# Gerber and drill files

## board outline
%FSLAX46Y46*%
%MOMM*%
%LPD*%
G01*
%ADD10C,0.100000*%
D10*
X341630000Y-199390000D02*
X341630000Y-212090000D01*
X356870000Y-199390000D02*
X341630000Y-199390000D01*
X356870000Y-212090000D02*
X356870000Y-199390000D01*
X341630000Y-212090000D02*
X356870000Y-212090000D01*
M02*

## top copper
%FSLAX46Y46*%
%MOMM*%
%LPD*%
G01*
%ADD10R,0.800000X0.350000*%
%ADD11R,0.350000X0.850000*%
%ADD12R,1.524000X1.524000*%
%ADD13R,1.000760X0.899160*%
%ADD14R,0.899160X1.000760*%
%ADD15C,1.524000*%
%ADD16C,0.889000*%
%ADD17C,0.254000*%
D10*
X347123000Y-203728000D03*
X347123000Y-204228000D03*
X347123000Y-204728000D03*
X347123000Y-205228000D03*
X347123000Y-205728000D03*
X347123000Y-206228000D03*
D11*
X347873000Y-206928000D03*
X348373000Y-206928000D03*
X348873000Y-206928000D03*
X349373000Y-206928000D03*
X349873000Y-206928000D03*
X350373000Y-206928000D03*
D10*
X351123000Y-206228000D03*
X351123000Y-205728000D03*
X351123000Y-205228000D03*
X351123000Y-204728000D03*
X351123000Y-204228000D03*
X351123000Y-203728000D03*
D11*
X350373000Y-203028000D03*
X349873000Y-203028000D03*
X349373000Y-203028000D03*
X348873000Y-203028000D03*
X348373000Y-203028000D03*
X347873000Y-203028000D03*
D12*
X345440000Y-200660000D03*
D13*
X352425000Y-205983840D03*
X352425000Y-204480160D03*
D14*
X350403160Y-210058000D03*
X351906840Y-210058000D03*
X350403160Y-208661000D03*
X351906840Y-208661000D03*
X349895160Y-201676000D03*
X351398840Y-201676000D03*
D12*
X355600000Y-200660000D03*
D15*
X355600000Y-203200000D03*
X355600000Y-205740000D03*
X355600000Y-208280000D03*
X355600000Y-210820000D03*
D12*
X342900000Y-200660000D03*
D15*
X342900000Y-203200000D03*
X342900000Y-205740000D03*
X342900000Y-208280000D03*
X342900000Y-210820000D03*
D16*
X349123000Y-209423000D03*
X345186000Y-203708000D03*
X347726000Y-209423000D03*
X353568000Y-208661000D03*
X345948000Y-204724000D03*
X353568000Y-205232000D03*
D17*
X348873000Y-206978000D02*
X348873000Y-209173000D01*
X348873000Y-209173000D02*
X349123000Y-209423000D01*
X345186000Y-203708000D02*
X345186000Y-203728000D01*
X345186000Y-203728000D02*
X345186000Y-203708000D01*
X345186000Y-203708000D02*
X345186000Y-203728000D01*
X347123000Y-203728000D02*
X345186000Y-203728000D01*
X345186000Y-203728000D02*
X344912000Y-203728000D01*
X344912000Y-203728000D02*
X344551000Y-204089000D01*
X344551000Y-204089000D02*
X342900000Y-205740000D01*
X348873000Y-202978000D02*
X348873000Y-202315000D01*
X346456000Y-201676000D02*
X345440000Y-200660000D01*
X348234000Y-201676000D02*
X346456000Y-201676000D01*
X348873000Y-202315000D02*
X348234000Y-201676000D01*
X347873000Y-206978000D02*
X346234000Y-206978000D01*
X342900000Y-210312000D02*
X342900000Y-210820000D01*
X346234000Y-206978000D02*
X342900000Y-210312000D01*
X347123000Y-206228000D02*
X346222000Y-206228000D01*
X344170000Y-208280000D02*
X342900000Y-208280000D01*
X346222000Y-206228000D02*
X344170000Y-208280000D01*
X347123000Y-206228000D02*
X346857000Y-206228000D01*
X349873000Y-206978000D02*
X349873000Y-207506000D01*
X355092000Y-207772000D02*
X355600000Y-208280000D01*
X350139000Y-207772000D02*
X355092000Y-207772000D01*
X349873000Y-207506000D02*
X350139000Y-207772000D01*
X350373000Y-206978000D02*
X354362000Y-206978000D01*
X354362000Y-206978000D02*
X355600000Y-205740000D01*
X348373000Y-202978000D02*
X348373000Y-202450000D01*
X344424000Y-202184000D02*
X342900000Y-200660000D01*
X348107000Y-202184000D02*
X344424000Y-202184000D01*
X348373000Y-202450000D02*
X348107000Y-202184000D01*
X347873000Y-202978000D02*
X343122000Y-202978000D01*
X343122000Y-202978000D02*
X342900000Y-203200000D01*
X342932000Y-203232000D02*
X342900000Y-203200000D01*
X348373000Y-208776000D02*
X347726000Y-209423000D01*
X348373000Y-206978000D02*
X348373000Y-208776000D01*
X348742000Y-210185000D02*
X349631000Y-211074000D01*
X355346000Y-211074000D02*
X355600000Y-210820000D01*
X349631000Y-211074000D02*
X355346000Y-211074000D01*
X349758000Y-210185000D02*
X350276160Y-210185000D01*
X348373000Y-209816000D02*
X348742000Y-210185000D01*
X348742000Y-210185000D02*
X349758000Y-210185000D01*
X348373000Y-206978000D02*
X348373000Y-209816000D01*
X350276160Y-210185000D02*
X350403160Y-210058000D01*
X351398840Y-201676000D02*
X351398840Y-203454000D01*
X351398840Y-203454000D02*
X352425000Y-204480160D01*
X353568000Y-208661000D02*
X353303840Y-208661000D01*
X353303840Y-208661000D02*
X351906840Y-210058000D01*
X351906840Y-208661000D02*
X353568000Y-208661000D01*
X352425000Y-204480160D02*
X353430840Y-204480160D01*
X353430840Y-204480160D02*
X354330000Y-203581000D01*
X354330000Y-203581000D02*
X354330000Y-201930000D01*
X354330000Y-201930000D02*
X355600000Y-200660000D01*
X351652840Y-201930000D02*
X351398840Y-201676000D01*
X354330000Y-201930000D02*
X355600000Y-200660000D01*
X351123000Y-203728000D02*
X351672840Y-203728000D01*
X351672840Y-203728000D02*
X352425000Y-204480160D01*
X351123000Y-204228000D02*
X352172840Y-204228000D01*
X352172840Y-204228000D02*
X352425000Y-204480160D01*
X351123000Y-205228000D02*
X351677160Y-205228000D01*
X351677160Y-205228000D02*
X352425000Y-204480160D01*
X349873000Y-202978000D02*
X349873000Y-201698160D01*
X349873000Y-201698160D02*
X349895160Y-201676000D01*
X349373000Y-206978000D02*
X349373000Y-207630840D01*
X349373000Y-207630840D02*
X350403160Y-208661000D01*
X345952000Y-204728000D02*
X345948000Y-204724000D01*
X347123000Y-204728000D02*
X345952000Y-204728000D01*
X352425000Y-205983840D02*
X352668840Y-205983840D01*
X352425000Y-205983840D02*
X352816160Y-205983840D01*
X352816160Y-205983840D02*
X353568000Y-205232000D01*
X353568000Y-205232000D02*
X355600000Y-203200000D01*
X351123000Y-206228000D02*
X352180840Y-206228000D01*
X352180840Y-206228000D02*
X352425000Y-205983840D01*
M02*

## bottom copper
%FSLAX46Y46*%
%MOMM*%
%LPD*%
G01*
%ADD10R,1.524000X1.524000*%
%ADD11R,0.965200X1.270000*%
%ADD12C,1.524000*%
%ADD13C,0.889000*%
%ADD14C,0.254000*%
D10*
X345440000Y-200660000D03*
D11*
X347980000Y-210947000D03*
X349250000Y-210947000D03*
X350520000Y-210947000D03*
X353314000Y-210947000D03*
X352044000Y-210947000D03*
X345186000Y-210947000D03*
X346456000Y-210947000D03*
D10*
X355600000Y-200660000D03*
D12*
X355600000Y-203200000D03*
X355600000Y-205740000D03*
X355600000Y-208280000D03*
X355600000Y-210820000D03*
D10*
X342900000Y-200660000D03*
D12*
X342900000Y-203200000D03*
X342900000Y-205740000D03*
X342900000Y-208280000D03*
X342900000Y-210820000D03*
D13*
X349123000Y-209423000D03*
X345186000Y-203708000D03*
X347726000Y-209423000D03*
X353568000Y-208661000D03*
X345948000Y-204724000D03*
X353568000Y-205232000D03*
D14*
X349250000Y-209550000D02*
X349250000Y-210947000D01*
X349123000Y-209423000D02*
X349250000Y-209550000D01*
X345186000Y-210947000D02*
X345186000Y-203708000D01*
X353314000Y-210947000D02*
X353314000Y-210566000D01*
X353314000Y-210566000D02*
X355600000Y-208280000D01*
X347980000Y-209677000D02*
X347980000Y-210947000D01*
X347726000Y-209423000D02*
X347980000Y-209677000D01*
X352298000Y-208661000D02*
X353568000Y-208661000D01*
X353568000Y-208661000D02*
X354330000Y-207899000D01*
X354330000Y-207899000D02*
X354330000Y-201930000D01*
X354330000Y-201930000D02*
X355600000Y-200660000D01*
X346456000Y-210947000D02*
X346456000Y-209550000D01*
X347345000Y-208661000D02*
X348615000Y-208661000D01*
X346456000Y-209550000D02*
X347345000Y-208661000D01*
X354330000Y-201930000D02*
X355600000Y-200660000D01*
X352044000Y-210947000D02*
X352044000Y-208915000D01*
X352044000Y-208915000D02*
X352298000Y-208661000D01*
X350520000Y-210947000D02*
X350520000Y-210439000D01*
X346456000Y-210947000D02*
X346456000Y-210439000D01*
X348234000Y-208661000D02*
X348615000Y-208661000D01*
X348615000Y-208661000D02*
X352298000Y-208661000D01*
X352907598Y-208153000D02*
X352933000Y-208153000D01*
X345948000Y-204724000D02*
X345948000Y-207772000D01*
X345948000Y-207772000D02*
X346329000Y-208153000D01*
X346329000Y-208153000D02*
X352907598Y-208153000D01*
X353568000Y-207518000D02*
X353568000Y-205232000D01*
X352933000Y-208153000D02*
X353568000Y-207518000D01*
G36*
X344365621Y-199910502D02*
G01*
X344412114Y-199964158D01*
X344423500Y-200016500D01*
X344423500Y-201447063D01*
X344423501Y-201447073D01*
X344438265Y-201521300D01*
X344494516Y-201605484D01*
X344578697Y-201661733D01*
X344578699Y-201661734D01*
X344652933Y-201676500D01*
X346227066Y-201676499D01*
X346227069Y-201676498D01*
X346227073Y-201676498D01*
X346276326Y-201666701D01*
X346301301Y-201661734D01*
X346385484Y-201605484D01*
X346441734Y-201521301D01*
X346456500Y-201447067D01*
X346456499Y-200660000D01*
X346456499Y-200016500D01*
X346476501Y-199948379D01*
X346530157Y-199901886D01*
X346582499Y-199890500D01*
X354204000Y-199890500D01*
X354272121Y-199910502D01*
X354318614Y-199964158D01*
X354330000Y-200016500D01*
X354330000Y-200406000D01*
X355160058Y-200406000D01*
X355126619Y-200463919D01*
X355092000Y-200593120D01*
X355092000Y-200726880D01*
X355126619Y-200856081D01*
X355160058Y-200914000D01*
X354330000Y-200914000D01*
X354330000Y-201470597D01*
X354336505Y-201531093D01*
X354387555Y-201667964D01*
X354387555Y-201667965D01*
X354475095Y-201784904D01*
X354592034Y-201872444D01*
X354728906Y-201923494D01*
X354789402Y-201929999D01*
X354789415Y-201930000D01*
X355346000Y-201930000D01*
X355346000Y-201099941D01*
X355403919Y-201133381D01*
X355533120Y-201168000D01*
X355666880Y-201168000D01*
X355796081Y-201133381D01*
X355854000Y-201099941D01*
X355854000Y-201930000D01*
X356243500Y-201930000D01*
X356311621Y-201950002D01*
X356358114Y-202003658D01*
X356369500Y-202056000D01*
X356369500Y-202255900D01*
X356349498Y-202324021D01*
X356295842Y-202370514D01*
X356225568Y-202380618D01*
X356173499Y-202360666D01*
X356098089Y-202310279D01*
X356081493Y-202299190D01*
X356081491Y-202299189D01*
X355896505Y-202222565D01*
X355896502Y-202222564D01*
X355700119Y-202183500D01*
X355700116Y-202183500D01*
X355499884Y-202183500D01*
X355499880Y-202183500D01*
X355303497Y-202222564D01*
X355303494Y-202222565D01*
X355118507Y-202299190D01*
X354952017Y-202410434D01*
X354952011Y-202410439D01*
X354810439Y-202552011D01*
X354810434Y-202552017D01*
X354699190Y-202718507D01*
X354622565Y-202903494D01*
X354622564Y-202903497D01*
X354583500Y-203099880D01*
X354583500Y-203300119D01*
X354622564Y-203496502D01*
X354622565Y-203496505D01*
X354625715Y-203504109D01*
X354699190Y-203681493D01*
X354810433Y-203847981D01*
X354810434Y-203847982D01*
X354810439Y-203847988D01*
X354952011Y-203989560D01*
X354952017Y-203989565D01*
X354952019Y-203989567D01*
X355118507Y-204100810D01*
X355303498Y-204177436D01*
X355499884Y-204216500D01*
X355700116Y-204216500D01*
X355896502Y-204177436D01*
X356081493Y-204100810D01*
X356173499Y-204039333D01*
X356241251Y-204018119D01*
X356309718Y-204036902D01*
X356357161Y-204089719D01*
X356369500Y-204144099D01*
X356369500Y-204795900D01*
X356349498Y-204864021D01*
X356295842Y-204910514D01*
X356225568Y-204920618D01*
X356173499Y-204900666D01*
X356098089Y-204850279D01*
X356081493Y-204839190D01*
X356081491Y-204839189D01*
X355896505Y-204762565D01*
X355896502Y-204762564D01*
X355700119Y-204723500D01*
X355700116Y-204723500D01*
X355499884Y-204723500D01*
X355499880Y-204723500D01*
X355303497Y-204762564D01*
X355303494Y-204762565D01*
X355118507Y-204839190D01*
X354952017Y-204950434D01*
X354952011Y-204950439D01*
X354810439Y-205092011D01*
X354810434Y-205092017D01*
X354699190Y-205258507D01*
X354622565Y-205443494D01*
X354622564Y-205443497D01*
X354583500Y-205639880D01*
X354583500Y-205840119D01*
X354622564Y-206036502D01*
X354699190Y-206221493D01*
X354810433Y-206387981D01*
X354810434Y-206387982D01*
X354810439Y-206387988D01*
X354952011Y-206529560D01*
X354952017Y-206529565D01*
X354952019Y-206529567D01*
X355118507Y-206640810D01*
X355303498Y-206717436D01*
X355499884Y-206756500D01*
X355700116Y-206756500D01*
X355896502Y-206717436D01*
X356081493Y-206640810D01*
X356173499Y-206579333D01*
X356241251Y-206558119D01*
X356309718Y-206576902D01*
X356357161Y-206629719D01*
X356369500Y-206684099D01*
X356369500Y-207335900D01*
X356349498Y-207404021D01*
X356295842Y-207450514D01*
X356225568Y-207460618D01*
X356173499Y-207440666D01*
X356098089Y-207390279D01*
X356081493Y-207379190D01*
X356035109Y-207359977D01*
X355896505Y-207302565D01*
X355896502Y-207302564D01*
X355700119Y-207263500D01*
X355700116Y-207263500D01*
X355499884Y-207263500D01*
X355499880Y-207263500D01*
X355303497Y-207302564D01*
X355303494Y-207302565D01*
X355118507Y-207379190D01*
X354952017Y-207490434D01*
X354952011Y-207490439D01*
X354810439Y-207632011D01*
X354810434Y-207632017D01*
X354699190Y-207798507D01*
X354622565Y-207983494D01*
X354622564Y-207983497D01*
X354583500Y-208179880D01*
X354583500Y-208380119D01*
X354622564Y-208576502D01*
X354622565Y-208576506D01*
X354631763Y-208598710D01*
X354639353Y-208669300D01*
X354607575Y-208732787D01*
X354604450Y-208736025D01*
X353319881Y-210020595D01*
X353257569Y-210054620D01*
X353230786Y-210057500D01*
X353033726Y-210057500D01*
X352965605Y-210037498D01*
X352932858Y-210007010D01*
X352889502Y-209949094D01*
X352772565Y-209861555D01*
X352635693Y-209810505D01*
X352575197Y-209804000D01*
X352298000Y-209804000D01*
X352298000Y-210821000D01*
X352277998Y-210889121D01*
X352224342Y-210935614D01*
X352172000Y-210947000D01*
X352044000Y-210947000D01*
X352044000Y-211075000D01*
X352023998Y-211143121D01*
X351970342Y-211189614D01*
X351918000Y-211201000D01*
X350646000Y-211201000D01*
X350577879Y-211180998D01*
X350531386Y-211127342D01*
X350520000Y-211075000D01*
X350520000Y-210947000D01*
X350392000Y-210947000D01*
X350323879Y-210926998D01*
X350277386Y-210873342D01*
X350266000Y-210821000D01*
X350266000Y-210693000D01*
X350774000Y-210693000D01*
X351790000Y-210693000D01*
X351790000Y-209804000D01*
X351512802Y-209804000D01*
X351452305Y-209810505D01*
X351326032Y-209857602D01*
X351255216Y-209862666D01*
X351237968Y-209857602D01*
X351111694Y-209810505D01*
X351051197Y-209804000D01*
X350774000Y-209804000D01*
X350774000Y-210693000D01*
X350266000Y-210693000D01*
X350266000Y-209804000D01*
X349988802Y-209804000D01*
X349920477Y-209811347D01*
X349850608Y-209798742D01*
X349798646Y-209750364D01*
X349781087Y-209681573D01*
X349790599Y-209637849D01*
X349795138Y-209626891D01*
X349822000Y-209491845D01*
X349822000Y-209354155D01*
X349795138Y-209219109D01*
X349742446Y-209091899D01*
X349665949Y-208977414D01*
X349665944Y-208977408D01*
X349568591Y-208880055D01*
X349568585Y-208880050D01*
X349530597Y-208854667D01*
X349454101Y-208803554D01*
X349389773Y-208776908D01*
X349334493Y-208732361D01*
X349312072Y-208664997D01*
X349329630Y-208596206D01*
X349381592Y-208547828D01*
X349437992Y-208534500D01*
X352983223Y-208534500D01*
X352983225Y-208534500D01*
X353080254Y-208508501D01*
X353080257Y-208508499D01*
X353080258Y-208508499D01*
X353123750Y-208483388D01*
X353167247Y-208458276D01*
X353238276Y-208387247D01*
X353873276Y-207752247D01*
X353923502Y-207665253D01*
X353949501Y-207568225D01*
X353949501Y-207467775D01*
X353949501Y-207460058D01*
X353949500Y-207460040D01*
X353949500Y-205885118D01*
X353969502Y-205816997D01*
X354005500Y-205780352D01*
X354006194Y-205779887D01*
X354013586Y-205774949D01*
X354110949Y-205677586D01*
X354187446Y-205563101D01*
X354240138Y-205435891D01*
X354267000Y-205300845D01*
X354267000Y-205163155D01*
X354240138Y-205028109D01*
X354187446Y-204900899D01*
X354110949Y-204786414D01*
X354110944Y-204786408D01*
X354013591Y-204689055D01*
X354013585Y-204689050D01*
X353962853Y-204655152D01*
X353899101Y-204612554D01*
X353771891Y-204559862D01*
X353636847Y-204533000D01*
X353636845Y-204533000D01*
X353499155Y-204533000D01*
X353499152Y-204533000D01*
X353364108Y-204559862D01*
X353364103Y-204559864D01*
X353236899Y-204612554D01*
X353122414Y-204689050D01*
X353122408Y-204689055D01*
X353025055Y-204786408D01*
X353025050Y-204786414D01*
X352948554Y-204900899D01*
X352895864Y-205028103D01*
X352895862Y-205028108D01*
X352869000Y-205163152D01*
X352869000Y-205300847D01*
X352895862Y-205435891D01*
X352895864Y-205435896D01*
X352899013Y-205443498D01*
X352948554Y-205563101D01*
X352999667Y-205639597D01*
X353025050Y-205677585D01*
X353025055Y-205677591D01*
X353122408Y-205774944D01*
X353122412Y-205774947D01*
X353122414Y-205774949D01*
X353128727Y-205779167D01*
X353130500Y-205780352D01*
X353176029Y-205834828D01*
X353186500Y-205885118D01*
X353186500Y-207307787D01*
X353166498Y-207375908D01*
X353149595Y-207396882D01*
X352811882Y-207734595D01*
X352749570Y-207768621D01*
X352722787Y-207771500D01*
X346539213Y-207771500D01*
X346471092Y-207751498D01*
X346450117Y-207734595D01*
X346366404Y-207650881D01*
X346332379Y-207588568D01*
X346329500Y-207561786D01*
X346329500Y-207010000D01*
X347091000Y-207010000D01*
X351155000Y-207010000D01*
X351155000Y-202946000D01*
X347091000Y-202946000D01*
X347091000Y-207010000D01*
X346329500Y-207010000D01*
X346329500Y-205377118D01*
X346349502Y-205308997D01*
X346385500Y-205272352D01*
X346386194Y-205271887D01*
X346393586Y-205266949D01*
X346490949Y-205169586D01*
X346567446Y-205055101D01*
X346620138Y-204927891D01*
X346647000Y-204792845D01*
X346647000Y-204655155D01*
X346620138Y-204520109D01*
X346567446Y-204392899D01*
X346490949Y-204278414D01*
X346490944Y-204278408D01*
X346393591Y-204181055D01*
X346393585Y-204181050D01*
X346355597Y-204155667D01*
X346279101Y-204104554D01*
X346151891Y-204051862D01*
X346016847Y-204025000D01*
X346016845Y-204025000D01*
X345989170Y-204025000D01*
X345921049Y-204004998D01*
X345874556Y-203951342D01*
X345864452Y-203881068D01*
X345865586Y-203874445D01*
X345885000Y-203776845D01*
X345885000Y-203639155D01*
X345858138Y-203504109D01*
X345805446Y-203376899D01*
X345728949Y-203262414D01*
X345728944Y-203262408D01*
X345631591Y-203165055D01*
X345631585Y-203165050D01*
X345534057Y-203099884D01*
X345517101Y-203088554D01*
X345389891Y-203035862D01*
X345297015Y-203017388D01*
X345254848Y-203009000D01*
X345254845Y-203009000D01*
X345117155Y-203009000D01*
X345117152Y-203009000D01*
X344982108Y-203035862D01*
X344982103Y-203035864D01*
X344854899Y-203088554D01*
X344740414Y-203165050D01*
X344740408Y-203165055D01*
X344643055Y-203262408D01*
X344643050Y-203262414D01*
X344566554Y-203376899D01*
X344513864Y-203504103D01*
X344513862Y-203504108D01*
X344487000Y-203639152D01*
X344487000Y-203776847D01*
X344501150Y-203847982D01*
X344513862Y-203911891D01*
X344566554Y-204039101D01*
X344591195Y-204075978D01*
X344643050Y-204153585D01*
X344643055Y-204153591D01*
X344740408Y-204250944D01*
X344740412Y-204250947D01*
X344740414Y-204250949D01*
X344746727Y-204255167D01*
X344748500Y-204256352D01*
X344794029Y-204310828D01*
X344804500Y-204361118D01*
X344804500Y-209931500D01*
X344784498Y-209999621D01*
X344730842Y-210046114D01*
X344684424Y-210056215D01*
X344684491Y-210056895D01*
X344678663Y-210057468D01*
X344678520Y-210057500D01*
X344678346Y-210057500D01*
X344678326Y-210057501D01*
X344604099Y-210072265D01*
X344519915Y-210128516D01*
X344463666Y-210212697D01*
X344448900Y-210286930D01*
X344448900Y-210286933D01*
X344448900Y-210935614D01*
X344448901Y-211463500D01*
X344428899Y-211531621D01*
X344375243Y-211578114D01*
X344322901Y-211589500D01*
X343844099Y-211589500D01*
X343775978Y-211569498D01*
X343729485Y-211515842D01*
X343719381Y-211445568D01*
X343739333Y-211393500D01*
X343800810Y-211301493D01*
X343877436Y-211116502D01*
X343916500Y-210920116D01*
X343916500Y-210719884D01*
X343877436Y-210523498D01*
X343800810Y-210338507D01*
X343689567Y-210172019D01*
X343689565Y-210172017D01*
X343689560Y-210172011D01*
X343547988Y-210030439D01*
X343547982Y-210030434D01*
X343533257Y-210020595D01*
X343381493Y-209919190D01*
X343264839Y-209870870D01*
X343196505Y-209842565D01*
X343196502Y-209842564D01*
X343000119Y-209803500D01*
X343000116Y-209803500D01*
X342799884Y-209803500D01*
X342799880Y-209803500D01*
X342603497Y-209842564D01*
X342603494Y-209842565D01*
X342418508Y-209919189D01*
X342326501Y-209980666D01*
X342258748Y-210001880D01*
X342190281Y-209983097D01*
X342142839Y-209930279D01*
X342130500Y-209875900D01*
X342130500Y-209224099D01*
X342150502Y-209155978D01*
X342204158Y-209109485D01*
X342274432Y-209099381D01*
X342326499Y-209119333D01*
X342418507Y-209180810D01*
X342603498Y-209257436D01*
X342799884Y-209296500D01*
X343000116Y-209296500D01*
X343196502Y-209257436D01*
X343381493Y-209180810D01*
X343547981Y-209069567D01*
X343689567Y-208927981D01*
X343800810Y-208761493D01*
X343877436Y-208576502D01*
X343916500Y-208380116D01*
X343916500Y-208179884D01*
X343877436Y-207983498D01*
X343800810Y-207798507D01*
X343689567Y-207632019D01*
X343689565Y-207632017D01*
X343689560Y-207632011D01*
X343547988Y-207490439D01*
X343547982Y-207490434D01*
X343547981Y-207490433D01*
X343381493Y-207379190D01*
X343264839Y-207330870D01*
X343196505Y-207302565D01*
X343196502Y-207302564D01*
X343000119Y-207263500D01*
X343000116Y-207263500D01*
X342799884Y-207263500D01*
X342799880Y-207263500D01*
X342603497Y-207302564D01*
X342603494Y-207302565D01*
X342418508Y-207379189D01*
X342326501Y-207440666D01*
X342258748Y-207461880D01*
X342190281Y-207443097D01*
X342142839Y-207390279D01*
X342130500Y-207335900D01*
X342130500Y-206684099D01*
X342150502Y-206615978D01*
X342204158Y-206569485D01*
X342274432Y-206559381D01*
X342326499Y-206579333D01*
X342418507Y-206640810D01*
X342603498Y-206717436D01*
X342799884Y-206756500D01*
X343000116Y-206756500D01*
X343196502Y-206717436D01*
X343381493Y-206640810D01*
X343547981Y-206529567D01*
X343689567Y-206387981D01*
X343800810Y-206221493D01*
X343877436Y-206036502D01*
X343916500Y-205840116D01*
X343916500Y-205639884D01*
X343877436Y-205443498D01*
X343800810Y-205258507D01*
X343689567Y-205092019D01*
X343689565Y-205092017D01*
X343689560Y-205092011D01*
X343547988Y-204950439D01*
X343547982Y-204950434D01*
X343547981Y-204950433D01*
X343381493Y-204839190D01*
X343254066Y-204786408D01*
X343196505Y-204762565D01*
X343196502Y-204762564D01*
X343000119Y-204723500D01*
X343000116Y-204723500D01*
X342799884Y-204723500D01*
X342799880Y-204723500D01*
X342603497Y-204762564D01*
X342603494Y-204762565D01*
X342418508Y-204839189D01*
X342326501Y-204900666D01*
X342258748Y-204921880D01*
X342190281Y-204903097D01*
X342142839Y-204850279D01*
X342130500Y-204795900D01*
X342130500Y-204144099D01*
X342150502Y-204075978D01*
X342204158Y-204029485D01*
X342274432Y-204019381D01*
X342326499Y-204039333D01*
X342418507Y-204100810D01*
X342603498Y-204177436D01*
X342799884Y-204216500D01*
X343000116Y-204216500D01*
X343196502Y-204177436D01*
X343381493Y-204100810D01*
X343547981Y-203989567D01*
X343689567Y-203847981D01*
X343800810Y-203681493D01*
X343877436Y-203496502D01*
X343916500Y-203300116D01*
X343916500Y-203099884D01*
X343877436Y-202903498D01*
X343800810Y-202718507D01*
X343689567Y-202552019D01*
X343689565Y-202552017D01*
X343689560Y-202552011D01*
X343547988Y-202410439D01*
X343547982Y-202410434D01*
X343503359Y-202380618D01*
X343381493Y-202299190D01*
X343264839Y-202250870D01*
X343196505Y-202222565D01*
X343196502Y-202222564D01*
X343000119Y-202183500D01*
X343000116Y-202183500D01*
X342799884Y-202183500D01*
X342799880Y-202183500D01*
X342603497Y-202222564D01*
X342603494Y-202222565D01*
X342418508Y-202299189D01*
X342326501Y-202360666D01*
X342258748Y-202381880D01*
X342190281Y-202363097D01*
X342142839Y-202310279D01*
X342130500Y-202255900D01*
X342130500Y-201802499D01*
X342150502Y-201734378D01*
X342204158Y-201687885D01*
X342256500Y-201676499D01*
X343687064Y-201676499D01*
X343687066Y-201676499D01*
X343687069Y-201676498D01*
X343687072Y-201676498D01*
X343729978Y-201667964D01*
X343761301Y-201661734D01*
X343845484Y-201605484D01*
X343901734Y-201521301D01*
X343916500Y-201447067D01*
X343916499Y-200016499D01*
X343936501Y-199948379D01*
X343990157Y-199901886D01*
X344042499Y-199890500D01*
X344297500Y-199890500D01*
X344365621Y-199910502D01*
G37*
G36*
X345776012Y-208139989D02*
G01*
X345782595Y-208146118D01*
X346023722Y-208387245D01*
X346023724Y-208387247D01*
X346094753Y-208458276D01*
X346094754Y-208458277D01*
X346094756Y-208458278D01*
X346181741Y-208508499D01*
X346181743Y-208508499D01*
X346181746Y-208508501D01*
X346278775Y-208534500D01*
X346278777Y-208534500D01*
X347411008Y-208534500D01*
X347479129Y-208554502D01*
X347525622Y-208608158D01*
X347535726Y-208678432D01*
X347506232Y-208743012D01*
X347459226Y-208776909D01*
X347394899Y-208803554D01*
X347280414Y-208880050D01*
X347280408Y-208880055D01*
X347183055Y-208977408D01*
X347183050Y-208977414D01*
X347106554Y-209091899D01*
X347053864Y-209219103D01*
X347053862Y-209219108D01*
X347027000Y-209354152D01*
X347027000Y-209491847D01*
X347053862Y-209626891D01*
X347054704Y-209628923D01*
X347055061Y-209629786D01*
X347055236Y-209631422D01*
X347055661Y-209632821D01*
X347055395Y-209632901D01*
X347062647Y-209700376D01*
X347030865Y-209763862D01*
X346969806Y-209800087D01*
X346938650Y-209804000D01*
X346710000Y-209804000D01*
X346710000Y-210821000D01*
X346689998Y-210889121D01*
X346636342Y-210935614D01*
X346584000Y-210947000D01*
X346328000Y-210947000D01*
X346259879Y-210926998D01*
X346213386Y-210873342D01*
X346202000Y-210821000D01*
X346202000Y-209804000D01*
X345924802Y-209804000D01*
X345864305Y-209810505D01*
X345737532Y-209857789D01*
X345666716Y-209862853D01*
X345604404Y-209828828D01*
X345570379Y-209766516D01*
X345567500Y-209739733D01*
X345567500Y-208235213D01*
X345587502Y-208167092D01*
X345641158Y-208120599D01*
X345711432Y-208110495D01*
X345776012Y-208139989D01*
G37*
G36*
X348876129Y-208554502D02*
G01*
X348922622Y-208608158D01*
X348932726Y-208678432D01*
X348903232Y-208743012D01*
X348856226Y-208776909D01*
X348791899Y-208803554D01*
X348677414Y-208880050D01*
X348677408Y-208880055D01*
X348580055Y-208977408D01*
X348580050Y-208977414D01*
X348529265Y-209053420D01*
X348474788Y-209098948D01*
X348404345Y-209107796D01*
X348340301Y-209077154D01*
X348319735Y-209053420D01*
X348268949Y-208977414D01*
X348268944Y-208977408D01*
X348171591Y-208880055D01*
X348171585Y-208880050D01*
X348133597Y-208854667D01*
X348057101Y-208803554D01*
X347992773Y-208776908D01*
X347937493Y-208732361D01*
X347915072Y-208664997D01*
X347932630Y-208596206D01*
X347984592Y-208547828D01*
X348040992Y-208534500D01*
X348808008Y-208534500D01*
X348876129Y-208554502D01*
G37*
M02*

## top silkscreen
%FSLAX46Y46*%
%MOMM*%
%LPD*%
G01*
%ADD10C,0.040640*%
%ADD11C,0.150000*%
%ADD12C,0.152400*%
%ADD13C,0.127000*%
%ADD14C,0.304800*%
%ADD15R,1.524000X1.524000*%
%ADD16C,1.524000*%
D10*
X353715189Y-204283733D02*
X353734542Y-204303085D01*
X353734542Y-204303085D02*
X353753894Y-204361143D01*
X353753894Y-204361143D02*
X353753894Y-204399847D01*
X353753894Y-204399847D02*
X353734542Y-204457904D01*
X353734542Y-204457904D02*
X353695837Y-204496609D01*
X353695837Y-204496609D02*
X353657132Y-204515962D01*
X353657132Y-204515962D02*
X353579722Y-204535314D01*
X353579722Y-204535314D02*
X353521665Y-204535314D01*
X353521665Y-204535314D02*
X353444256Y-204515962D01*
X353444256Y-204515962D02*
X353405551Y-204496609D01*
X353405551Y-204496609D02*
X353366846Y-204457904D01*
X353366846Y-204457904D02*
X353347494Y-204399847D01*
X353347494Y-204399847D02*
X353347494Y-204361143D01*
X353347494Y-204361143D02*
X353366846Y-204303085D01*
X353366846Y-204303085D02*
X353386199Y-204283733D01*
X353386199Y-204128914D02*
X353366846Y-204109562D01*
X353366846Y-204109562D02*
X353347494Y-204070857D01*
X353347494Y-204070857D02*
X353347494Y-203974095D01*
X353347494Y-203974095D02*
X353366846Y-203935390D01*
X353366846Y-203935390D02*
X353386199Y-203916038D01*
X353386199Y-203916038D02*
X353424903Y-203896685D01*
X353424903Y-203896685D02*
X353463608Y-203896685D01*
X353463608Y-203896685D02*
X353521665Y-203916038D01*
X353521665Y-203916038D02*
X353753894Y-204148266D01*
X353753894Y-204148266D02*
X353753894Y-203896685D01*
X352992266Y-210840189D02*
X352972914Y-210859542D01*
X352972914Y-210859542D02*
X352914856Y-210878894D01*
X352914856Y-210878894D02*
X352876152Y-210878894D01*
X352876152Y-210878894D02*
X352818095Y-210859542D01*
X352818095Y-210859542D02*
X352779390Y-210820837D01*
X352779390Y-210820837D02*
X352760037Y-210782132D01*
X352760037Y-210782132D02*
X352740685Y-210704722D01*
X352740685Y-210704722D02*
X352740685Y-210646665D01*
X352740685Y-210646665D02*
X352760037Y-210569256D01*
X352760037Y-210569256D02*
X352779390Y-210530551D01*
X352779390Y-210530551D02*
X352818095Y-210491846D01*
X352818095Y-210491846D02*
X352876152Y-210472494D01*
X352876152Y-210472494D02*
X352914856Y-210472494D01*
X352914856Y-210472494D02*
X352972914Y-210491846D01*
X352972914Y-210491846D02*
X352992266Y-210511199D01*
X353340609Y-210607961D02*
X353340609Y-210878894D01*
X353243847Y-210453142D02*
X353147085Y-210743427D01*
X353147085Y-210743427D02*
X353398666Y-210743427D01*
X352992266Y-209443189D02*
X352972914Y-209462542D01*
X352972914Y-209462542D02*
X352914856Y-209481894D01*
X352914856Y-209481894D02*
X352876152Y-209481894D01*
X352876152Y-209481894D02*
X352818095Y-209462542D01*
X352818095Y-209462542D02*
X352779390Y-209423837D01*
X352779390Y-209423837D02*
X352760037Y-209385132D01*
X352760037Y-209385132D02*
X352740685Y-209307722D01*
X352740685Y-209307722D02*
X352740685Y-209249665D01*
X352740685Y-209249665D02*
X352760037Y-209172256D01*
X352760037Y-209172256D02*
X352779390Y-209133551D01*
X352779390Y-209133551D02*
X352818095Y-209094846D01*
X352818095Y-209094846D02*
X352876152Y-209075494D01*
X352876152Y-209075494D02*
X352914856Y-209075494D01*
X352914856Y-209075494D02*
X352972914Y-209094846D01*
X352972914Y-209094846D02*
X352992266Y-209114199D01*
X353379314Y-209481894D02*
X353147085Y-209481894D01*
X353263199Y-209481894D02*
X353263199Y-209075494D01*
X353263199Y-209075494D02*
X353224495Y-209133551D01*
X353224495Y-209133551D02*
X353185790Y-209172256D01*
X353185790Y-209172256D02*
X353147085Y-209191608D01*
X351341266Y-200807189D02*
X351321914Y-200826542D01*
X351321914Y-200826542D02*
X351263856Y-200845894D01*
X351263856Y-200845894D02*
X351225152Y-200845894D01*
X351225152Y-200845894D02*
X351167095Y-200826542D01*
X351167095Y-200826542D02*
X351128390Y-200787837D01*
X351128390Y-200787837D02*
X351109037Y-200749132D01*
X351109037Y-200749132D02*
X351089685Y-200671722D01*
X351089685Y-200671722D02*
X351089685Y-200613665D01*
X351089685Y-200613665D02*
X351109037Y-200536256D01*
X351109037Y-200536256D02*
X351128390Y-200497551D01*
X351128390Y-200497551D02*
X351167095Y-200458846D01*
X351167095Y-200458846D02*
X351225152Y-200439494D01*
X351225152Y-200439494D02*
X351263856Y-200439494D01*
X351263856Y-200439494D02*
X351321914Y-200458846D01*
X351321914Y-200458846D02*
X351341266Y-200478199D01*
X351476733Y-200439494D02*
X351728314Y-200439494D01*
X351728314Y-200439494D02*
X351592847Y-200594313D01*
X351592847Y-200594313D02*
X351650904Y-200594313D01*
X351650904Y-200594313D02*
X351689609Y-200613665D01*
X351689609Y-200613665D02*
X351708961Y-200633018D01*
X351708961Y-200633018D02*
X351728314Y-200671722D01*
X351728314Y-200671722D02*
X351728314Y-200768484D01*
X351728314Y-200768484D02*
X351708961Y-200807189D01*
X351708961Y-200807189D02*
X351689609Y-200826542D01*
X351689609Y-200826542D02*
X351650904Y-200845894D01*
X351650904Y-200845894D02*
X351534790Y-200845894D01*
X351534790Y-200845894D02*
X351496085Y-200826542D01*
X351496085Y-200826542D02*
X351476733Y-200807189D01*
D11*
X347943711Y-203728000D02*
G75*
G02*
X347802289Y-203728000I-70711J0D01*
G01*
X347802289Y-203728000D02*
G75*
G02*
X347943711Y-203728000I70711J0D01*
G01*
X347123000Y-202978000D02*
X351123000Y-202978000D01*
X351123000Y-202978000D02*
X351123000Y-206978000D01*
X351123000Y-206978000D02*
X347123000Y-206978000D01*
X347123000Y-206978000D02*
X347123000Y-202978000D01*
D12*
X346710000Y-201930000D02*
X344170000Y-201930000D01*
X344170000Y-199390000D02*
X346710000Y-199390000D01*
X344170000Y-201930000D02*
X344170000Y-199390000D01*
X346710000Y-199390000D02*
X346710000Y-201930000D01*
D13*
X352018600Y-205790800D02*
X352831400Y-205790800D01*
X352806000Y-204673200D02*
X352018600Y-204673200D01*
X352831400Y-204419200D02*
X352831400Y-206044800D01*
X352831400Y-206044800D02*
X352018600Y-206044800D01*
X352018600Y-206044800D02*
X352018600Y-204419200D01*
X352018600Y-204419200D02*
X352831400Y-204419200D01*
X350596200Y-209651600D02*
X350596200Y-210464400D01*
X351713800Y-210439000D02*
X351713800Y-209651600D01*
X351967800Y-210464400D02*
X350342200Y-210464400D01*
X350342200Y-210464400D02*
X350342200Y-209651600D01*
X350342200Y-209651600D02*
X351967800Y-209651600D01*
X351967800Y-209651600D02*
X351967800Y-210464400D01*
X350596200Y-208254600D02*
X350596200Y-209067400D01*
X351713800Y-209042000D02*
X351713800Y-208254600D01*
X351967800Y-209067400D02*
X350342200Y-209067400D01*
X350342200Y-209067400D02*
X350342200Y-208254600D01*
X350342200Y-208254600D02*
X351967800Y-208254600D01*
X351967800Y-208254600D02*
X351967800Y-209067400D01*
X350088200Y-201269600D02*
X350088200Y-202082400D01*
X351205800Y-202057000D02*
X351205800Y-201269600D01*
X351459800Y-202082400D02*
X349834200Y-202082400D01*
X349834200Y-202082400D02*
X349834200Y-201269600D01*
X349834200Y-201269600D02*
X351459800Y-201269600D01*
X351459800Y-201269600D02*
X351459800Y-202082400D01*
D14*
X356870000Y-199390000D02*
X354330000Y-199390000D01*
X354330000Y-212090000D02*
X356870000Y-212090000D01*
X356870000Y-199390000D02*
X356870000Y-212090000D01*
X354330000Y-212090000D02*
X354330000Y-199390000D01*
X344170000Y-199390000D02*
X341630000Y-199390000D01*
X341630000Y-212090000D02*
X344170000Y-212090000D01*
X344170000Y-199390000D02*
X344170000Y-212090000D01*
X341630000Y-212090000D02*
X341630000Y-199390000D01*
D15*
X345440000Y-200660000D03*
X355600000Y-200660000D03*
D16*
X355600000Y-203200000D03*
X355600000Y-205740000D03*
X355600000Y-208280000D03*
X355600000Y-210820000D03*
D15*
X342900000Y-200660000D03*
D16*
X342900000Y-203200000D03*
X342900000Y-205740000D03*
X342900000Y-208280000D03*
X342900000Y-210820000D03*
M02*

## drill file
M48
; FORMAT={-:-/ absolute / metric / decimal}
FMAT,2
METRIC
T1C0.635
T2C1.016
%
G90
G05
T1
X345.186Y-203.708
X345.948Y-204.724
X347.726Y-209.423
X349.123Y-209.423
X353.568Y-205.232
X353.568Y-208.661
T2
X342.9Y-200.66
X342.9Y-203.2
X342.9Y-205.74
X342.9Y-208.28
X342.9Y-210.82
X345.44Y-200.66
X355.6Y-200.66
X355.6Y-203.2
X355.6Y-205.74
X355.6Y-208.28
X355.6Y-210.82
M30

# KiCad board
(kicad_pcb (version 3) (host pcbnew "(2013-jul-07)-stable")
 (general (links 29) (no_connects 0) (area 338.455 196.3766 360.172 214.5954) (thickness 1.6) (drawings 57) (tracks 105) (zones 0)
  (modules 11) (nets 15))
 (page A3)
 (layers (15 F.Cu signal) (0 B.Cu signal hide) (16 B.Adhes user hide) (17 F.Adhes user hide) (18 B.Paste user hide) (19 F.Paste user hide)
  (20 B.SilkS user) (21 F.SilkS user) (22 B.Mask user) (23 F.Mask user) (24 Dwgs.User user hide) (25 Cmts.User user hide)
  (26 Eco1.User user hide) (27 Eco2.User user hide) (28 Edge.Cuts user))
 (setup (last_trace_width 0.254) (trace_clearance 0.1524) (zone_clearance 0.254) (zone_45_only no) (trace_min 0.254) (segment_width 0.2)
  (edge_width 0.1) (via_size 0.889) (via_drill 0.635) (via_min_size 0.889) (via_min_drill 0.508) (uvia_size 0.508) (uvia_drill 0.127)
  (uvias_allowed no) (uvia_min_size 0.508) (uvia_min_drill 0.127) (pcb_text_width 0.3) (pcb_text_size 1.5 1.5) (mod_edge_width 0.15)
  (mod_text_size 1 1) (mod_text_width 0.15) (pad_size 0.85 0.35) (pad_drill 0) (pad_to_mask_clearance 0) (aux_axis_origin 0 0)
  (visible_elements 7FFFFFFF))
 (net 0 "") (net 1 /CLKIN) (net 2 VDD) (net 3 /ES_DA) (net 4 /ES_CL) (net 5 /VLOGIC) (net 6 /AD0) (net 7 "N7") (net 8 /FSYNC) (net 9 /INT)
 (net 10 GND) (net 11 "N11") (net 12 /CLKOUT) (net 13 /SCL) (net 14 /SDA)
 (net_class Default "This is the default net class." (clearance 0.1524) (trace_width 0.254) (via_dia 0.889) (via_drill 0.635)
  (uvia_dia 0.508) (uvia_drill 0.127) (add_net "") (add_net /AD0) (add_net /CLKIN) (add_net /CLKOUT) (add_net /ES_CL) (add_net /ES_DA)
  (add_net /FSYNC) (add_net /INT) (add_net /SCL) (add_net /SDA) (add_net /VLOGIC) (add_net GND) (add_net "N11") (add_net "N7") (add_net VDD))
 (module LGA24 (layer F.Cu) (at 349.123 204.978)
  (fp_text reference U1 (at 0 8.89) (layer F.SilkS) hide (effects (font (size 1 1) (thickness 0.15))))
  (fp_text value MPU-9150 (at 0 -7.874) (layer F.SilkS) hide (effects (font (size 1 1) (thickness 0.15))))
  (fp_circle (center -1.25 -1.25) (end -1.2 -1.2) (layer F.SilkS) (width 0.15))
  (fp_line (start -2 -2) (end 2 -2) (layer F.SilkS) (width 0.15))
  (fp_line (start 2 -2) (end 2 2) (layer F.SilkS) (width 0.15))
  (fp_line (start 2 2) (end -2 2) (layer F.SilkS) (width 0.15))
  (fp_line (start -2 2) (end -2 -2) (layer F.SilkS) (width 0.15))
  (pad 1 smd rect (at -2 -1.25) (size 0.8 0.35) (layers F.Cu F.Paste F.Mask) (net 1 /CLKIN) (clearance 0.0762))
  (pad 2 smd rect (at -2 -0.75) (size 0.8 0.35) (layers F.Cu F.Paste F.Mask) (clearance 0.0762))
  (pad 3 smd rect (at -2 -0.25) (size 0.8 0.35) (layers F.Cu F.Paste F.Mask) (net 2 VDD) (clearance 0.0762))
  (pad 4 smd rect (at -2 0.25) (size 0.8 0.35) (layers F.Cu F.Paste F.Mask) (clearance 0.0762))
  (pad 5 smd rect (at -2 0.75) (size 0.8 0.35) (layers F.Cu F.Paste F.Mask) (clearance 0.0762))
  (pad 6 smd rect (at -2 1.25) (size 0.8 0.35) (layers F.Cu F.Paste F.Mask) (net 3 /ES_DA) (clearance 0.0762))
  (pad 7 smd rect (at -1.25 2 90) (size 0.85 0.35) (drill (offset 0.05 0)) (layers F.Cu F.Paste F.Mask) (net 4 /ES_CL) (clearance 0.0762))
  (pad 8 smd rect (at -0.75 2 90) (size 0.85 0.35) (drill (offset 0.05 0)) (layers F.Cu F.Paste F.Mask) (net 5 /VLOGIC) (clearance 0.0762))
  (pad 9 smd rect (at -0.25 2 90) (size 0.85 0.35) (drill (offset 0.05 0)) (layers F.Cu F.Paste F.Mask) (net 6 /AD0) (clearance 0.0762))
  (pad 10 smd rect (at 0.25 2 90) (size 0.85 0.35) (drill (offset 0.05 0)) (layers F.Cu F.Paste F.Mask) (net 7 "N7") (clearance 0.0762))
  (pad 11 smd rect (at 0.75 2 90) (size 0.85 0.35) (drill (offset 0.05 0)) (layers F.Cu F.Paste F.Mask) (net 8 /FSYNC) (clearance 0.0762))
  (pad 12 smd rect (at 1.25 2 90) (size 0.85 0.35) (drill (offset 0.05 0)) (layers F.Cu F.Paste F.Mask) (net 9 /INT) (clearance 0.0762))
  (pad 13 smd rect (at 2 1.25) (size 0.8 0.35) (layers F.Cu F.Paste F.Mask) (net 2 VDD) (clearance 0.0762))
  (pad 14 smd rect (at 2 0.75) (size 0.8 0.35) (layers F.Cu F.Paste F.Mask) (clearance 0.0762))
  (pad 15 smd rect (at 2 0.25) (size 0.8 0.35) (layers F.Cu F.Paste F.Mask) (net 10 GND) (clearance 0.0762))
  (pad 16 smd rect (at 2 -0.25) (size 0.8 0.35) (layers F.Cu F.Paste F.Mask) (clearance 0.0762))
  (pad 17 smd rect (at 2 -0.75) (size 0.8 0.35) (layers F.Cu F.Paste F.Mask) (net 10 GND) (clearance 0.0762))
  (pad 18 smd rect (at 2 -1.25) (size 0.8 0.35) (layers F.Cu F.Paste F.Mask) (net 10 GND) (clearance 0.0762))
  (pad 19 smd rect (at 1.25 -2 270) (size 0.85 0.35) (drill (offset 0.05 0)) (layers F.Cu F.Paste F.Mask) (clearance 0.0762))
  (pad 20 smd rect (at 0.75 -2 270) (size 0.85 0.35) (drill (offset 0.05 0)) (layers F.Cu F.Paste F.Mask) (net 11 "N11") (clearance 0.0762))
  (pad 21 smd rect (at 0.25 -2 270) (size 0.85 0.35) (drill (offset 0.05 0)) (layers F.Cu F.Paste F.Mask) (clearance 0.0762))
  (pad 22 smd rect (at -0.25 -2 270) (size 0.85 0.35) (drill (offset 0.05 0)) (layers F.Cu F.Paste F.Mask) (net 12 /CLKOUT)
   (clearance 0.0762))
  (pad 23 smd rect (at -0.75 -2 270) (size 0.85 0.35) (drill (offset 0.05 0)) (layers F.Cu F.Paste F.Mask) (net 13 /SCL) (clearance 0.0762))
  (pad 24 smd rect (at -1.25 -2 270) (size 0.85 0.35) (drill (offset 0.05 0)) (layers F.Cu F.Paste F.Mask) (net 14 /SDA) (clearance 0.0762)))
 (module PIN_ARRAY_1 (layer F.Cu) (at 345.44 200.66)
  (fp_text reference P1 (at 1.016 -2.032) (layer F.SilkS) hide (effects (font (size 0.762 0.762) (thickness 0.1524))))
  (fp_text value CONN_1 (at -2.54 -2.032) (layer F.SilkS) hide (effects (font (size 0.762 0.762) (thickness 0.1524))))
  (fp_line (start 1.27 1.27) (end -1.27 1.27) (layer F.SilkS) (width 0.1524))
  (fp_line (start -1.27 -1.27) (end 1.27 -1.27) (layer F.SilkS) (width 0.1524))
  (fp_line (start -1.27 1.27) (end -1.27 -1.27) (layer F.SilkS) (width 0.1524))
  (fp_line (start 1.27 -1.27) (end 1.27 1.27) (layer F.SilkS) (width 0.1524))
  (pad 1 thru_hole rect (at 0 0) (size 1.524 1.524) (drill 1.016) (layers *.Cu *.Mask F.SilkS) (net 12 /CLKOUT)))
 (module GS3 (layer B.Cu) (at 349.25 210.947 270)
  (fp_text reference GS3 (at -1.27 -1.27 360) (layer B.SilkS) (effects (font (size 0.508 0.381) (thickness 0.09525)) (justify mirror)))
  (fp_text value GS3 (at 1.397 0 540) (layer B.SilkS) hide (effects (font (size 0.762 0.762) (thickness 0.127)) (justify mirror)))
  (pad 1 smd rect (at 0 1.27 270) (size 1.27 0.9652) (layers B.Cu B.Paste B.Mask) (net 5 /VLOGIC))
  (pad 2 smd rect (at 0 0 270) (size 1.27 0.9652) (layers B.Cu B.Paste B.Mask) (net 6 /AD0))
  (pad 3 smd rect (at 0 -1.27 270) (size 1.27 0.9652) (layers B.Cu B.Paste B.Mask) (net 10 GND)))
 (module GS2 (layer B.Cu) (at 352.679 210.947 90)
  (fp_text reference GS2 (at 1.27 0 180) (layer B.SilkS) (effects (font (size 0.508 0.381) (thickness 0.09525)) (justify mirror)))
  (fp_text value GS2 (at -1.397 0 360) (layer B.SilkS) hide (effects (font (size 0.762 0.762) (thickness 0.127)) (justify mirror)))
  (pad 1 smd rect (at 0 0.635 90) (size 1.27 0.9652) (layers B.Cu B.Paste B.Mask) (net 8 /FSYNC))
  (pad 2 smd rect (at 0 -0.635 90) (size 1.27 0.9652) (layers B.Cu B.Paste B.Mask) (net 10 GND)))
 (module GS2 (layer B.Cu) (at 345.821 210.947 270)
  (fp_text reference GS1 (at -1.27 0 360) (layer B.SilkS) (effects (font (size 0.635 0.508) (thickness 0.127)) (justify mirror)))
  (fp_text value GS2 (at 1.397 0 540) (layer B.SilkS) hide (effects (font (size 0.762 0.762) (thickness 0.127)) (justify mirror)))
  (pad 1 smd rect (at 0 0.635 270) (size 1.27 0.9652) (layers B.Cu B.Paste B.Mask) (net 1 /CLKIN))
  (pad 2 smd rect (at 0 -0.635 270) (size 1.27 0.9652) (layers B.Cu B.Paste B.Mask) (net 10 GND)))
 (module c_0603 (layer F.Cu) (at 352.425 205.232 270)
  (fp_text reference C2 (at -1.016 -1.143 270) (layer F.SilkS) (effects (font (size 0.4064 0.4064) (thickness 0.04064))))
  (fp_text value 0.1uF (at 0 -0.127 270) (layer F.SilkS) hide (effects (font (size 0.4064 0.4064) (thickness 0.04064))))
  (fp_line (start 0.5588 0.4064) (end 0.5588 -0.4064) (layer F.SilkS) (width 0.127))
  (fp_line (start -0.5588 -0.381) (end -0.5588 0.4064) (layer F.SilkS) (width 0.127))
  (fp_line (start -0.8128 -0.4064) (end 0.8128 -0.4064) (layer F.SilkS) (width 0.127))
  (fp_line (start 0.8128 -0.4064) (end 0.8128 0.4064) (layer F.SilkS) (width 0.127))
  (fp_line (start 0.8128 0.4064) (end -0.8128 0.4064) (layer F.SilkS) (width 0.127))
  (fp_line (start -0.8128 0.4064) (end -0.8128 -0.4064) (layer F.SilkS) (width 0.127))
  (pad 1 smd rect (at 0.75184 0 270) (size 0.89916 1.00076) (layers F.Cu F.Paste F.Mask) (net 2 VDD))
  (pad 2 smd rect (at -0.75184 0 270) (size 0.89916 1.00076) (layers F.Cu F.Paste F.Mask) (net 10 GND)))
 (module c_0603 (layer F.Cu) (at 351.155 210.058 180)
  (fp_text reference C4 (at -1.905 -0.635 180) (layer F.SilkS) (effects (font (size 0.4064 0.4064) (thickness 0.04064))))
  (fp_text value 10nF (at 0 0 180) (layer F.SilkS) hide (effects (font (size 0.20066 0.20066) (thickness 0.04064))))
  (fp_line (start 0.5588 0.4064) (end 0.5588 -0.4064) (layer F.SilkS) (width 0.127))
  (fp_line (start -0.5588 -0.381) (end -0.5588 0.4064) (layer F.SilkS) (width 0.127))
  (fp_line (start -0.8128 -0.4064) (end 0.8128 -0.4064) (layer F.SilkS) (width 0.127))
  (fp_line (start 0.8128 -0.4064) (end 0.8128 0.4064) (layer F.SilkS) (width 0.127))
  (fp_line (start 0.8128 0.4064) (end -0.8128 0.4064) (layer F.SilkS) (width 0.127))
  (fp_line (start -0.8128 0.4064) (end -0.8128 -0.4064) (layer F.SilkS) (width 0.127))
  (pad 1 smd rect (at 0.75184 0 180) (size 0.89916 1.00076) (layers F.Cu F.Paste F.Mask) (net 5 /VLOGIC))
  (pad 2 smd rect (at -0.75184 0 180) (size 0.89916 1.00076) (layers F.Cu F.Paste F.Mask) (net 10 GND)))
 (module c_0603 (layer F.Cu) (at 351.155 208.661 180)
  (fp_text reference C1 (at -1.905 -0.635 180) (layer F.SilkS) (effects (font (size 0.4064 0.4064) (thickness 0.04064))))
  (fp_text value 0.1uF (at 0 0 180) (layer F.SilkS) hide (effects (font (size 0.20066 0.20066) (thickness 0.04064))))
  (fp_line (start 0.5588 0.4064) (end 0.5588 -0.4064) (layer F.SilkS) (width 0.127))
  (fp_line (start -0.5588 -0.381) (end -0.5588 0.4064) (layer F.SilkS) (width 0.127))
  (fp_line (start -0.8128 -0.4064) (end 0.8128 -0.4064) (layer F.SilkS) (width 0.127))
  (fp_line (start 0.8128 -0.4064) (end 0.8128 0.4064) (layer F.SilkS) (width 0.127))
  (fp_line (start 0.8128 0.4064) (end -0.8128 0.4064) (layer F.SilkS) (width 0.127))
  (fp_line (start -0.8128 0.4064) (end -0.8128 -0.4064) (layer F.SilkS) (width 0.127))
  (pad 1 smd rect (at 0.75184 0 180) (size 0.89916 1.00076) (layers F.Cu F.Paste F.Mask) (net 7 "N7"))
  (pad 2 smd rect (at -0.75184 0 180) (size 0.89916 1.00076) (layers F.Cu F.Paste F.Mask) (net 10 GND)))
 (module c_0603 (layer F.Cu) (at 350.647 201.676 180)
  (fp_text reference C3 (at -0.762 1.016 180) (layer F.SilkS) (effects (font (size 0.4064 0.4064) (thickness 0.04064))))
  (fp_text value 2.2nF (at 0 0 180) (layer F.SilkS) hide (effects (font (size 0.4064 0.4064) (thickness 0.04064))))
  (fp_line (start 0.5588 0.4064) (end 0.5588 -0.4064) (layer F.SilkS) (width 0.127))
  (fp_line (start -0.5588 -0.381) (end -0.5588 0.4064) (layer F.SilkS) (width 0.127))
  (fp_line (start -0.8128 -0.4064) (end 0.8128 -0.4064) (layer F.SilkS) (width 0.127))
  (fp_line (start 0.8128 -0.4064) (end 0.8128 0.4064) (layer F.SilkS) (width 0.127))
  (fp_line (start 0.8128 0.4064) (end -0.8128 0.4064) (layer F.SilkS) (width 0.127))
  (fp_line (start -0.8128 0.4064) (end -0.8128 -0.4064) (layer F.SilkS) (width 0.127))
  (pad 1 smd rect (at 0.75184 0 180) (size 0.89916 1.00076) (layers F.Cu F.Paste F.Mask) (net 11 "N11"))
  (pad 2 smd rect (at -0.75184 0 180) (size 0.89916 1.00076) (layers F.Cu F.Paste F.Mask) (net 10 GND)))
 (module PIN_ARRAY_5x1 (layer F.Cu) (at 355.6 205.74 270)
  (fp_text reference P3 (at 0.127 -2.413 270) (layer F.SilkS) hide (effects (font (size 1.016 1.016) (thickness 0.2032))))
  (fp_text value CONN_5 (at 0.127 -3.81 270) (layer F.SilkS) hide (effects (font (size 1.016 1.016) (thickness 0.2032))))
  (fp_line (start -6.35 -1.27) (end -6.35 1.27) (layer F.SilkS) (width 0.3048))
  (fp_line (start 6.35 1.27) (end 6.35 -1.27) (layer F.SilkS) (width 0.3048))
  (fp_line (start -6.35 -1.27) (end 6.35 -1.27) (layer F.SilkS) (width 0.3048))
  (fp_line (start 6.35 1.27) (end -6.35 1.27) (layer F.SilkS) (width 0.3048))
  (pad 1 thru_hole rect (at -5.08 0 270) (size 1.524 1.524) (drill 1.016) (layers *.Cu *.Mask F.SilkS) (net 10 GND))
  (pad 2 thru_hole circle (at -2.54 0 270) (size 1.524 1.524) (drill 1.016) (layers *.Cu *.Mask F.SilkS) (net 2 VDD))
  (pad 3 thru_hole circle (at 0 0 270) (size 1.524 1.524) (drill 1.016) (layers *.Cu *.Mask F.SilkS) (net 9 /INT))
  (pad 4 thru_hole circle (at 2.54 0 270) (size 1.524 1.524) (drill 1.016) (layers *.Cu *.Mask F.SilkS) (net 8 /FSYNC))
  (pad 5 thru_hole circle (at 5.08 0 270) (size 1.524 1.524) (drill 1.016) (layers *.Cu *.Mask F.SilkS) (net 5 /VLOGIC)))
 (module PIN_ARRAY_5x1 (layer F.Cu) (at 342.9 205.74 270)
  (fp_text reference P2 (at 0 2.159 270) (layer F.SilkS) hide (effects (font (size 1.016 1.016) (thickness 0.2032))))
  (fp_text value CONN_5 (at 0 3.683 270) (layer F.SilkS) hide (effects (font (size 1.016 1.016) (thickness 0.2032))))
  (fp_line (start -6.35 -1.27) (end -6.35 1.27) (layer F.SilkS) (width 0.3048))
  (fp_line (start 6.35 1.27) (end 6.35 -1.27) (layer F.SilkS) (width 0.3048))
  (fp_line (start -6.35 -1.27) (end 6.35 -1.27) (layer F.SilkS) (width 0.3048))
  (fp_line (start 6.35 1.27) (end -6.35 1.27) (layer F.SilkS) (width 0.3048))
  (pad 1 thru_hole rect (at -5.08 0 270) (size 1.524 1.524) (drill 1.016) (layers *.Cu *.Mask F.SilkS) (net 13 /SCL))
  (pad 2 thru_hole circle (at -2.54 0 270) (size 1.524 1.524) (drill 1.016) (layers *.Cu *.Mask F.SilkS) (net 14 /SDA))
  (pad 3 thru_hole circle (at 0 0 270) (size 1.524 1.524) (drill 1.016) (layers *.Cu *.Mask F.SilkS) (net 1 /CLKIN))
  (pad 4 thru_hole circle (at 2.54 0 270) (size 1.524 1.524) (drill 1.016) (layers *.Cu *.Mask F.SilkS) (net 3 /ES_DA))
  (pad 5 thru_hole circle (at 5.08 0 270) (size 1.524 1.524) (drill 1.016) (layers *.Cu *.Mask F.SilkS) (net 4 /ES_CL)))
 (gr_line (start 341.63 199.39) (end 341.63 212.09) (angle 90) (layer Edge.Cuts) (width 0.1))
 (gr_line (start 356.87 199.39) (end 341.63 199.39) (angle 90) (layer Edge.Cuts) (width 0.1))
 (gr_line (start 356.87 212.09) (end 356.87 199.39) (angle 90) (layer Edge.Cuts) (width 0.1))
 (gr_line (start 341.63 212.09) (end 356.87 212.09) (angle 90) (layer Edge.Cuts) (width 0.1))
 (segment (start 348.873 206.978) (end 348.873 209.173) (width 0.254) (layer F.Cu) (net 6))
 (segment (start 349.25 209.55) (end 349.25 210.947) (width 0.254) (layer B.Cu) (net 6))
 (segment (start 349.123 209.423) (end 349.25 209.55) (width 0.254) (layer B.Cu) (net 6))
 (via (at 349.123 209.423) (size 0.889) (layers F.Cu B.Cu) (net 6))
 (segment (start 348.873 209.173) (end 349.123 209.423) (width 0.254) (layer F.Cu) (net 6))
 (segment (start 345.186 210.947) (end 345.186 203.708) (width 0.254) (layer B.Cu) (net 1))
 (via (at 345.186 203.708) (size 0.889) (layers F.Cu B.Cu) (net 1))
 (segment (start 345.186 203.708) (end 345.186 203.728) (width 0.254) (layer F.Cu) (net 1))
 (segment (start 345.186 203.728) (end 345.186 203.708) (width 0.254) (layer F.Cu) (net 1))
 (segment (start 345.186 203.708) (end 345.186 203.728) (width 0.254) (layer F.Cu) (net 1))
 (segment (start 347.123 203.728) (end 345.186 203.728) (width 0.254) (layer F.Cu) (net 1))
 (segment (start 345.186 203.728) (end 344.912 203.728) (width 0.254) (layer F.Cu) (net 1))
 (segment (start 344.912 203.728) (end 344.551 204.089) (width 0.254) (layer F.Cu) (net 1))
 (segment (start 344.551 204.089) (end 342.9 205.74) (width 0.254) (layer F.Cu) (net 1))
 (segment (start 348.873 202.978) (end 348.873 202.315) (width 0.254) (layer F.Cu) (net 12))
 (segment (start 346.456 201.676) (end 345.44 200.66) (width 0.254) (layer F.Cu) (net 12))
 (segment (start 348.234 201.676) (end 346.456 201.676) (width 0.254) (layer F.Cu) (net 12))
 (segment (start 348.873 202.315) (end 348.234 201.676) (width 0.254) (layer F.Cu) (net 12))
 (segment (start 347.873 206.978) (end 346.234 206.978) (width 0.254) (layer F.Cu) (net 4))
 (segment (start 342.9 210.312) (end 342.9 210.82) (width 0.254) (layer F.Cu) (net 4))
 (segment (start 346.234 206.978) (end 342.9 210.312) (width 0.254) (layer F.Cu) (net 4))
 (segment (start 347.123 206.228) (end 346.222 206.228) (width 0.254) (layer F.Cu) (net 3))
 (segment (start 344.17 208.28) (end 342.9 208.28) (width 0.254) (layer F.Cu) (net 3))
 (segment (start 346.222 206.228) (end 344.17 208.28) (width 0.254) (layer F.Cu) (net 3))
 (segment (start 347.123 206.228) (end 346.857 206.228) (width 0.254) (layer F.Cu) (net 3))
 (segment (start 353.314 210.947) (end 353.314 210.566) (width 0.254) (layer B.Cu) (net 8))
 (segment (start 353.314 210.566) (end 355.6 208.28) (width 0.254) (layer B.Cu) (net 8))
 (segment (start 349.873 206.978) (end 349.873 207.506) (width 0.254) (layer F.Cu) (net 8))
 (segment (start 355.092 207.772) (end 355.6 208.28) (width 0.254) (layer F.Cu) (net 8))
 (segment (start 350.139 207.772) (end 355.092 207.772) (width 0.254) (layer F.Cu) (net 8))
 (segment (start 349.873 207.506) (end 350.139 207.772) (width 0.254) (layer F.Cu) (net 8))
 (segment (start 350.373 206.978) (end 354.362 206.978) (width 0.254) (layer F.Cu) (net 9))
 (segment (start 354.362 206.978) (end 355.6 205.74) (width 0.254) (layer F.Cu) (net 9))
 (segment (start 348.373 202.978) (end 348.373 202.45) (width 0.254) (layer F.Cu) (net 13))
 (segment (start 344.424 202.184) (end 342.9 200.66) (width 0.254) (layer F.Cu) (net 13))
 (segment (start 348.107 202.184) (end 344.424 202.184) (width 0.254) (layer F.Cu) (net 13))
 (segment (start 348.373 202.45) (end 348.107 202.184) (width 0.254) (layer F.Cu) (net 13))
 (segment (start 347.873 202.978) (end 343.122 202.978) (width 0.254) (layer F.Cu) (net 14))
 (segment (start 343.122 202.978) (end 342.9 203.2) (width 0.254) (layer F.Cu) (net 14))
 (segment (start 342.932 203.232) (end 342.9 203.2) (width 0.254) (layer F.Cu) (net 14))
 (via (at 347.726 209.423) (size 0.889) (layers F.Cu B.Cu) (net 5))
 (segment (start 348.373 208.776) (end 347.726 209.423) (width 0.254) (layer F.Cu) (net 5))
 (segment (start 348.373 206.978) (end 348.373 208.776) (width 0.254) (layer F.Cu) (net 5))
 (segment (start 347.98 209.677) (end 347.98 210.947) (width 0.254) (layer B.Cu) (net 5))
 (segment (start 347.726 209.423) (end 347.98 209.677) (width 0.254) (layer B.Cu) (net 5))
 (segment (start 348.742 210.185) (end 349.631 211.074) (width 0.254) (layer F.Cu) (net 5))
 (segment (start 355.346 211.074) (end 355.6 210.82) (width 0.254) (layer F.Cu) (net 5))
 (segment (start 349.631 211.074) (end 355.346 211.074) (width 0.254) (layer F.Cu) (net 5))
 (segment (start 349.758 210.185) (end 350.27616 210.185) (width 0.254) (layer F.Cu) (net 5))
 (segment (start 348.373 209.816) (end 348.742 210.185) (width 0.254) (layer F.Cu) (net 5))
 (segment (start 348.742 210.185) (end 349.758 210.185) (width 0.254) (layer F.Cu) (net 5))
 (segment (start 348.373 206.978) (end 348.373 209.816) (width 0.254) (layer F.Cu) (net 5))
 (segment (start 350.27616 210.185) (end 350.40316 210.058) (width 0.254) (layer F.Cu) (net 5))
 (segment (start 351.39884 201.676) (end 351.39884 203.454) (width 0.254) (layer F.Cu) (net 10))
 (segment (start 351.39884 203.454) (end 352.425 204.48016) (width 0.254) (layer F.Cu) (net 10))
 (segment (start 352.298 208.661) (end 353.568 208.661) (width 0.254) (layer B.Cu) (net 10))
 (segment (start 353.568 208.661) (end 354.33 207.899) (width 0.254) (layer B.Cu) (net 10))
 (segment (start 354.33 207.899) (end 354.33 201.93) (width 0.254) (layer B.Cu) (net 10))
 (segment (start 354.33 201.93) (end 355.6 200.66) (width 0.254) (layer B.Cu) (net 10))
 (segment (start 353.568 208.661) (end 353.30384 208.661) (width 0.254) (layer F.Cu) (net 10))
 (segment (start 353.30384 208.661) (end 351.90684 210.058) (width 0.254) (layer F.Cu) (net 10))
 (via (at 353.568 208.661) (size 0.889) (layers F.Cu B.Cu) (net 10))
 (segment (start 351.90684 208.661) (end 353.568 208.661) (width 0.254) (layer F.Cu) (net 10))
 (segment (start 346.456 210.947) (end 346.456 209.55) (width 0.254) (layer B.Cu) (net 10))
 (segment (start 347.345 208.661) (end 348.615 208.661) (width 0.254) (layer B.Cu) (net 10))
 (segment (start 346.456 209.55) (end 347.345 208.661) (width 0.254) (layer B.Cu) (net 10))
 (segment (start 352.425 204.48016) (end 353.43084 204.48016) (width 0.254) (layer F.Cu) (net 10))
 (segment (start 353.43084 204.48016) (end 354.33 203.581) (width 0.254) (layer F.Cu) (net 10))
 (segment (start 354.33 203.581) (end 354.33 201.93) (width 0.254) (layer F.Cu) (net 10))
 (segment (start 354.33 201.93) (end 355.6 200.66) (width 0.254) (layer F.Cu) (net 10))
 (segment (start 354.33 201.93) (end 355.6 200.66) (width 0.254) (layer B.Cu) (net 10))
 (segment (start 351.65284 201.93) (end 351.39884 201.676) (width 0.254) (layer F.Cu) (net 10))
 (segment (start 354.33 201.93) (end 355.6 200.66) (width 0.254) (layer F.Cu) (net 10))
 (segment (start 352.044 210.947) (end 352.044 208.915) (width 0.254) (layer B.Cu) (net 10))
 (segment (start 352.044 208.915) (end 352.298 208.661) (width 0.254) (layer B.Cu) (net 10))
 (segment (start 350.52 210.947) (end 350.52 210.439) (width 0.254) (layer B.Cu) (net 10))
 (segment (start 346.456 210.947) (end 346.456 210.439) (width 0.254) (layer B.Cu) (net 10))
 (segment (start 348.234 208.661) (end 348.615 208.661) (width 0.254) (layer B.Cu) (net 10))
 (segment (start 348.615 208.661) (end 352.298 208.661) (width 0.254) (layer B.Cu) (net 10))
 (segment (start 351.123 203.728) (end 351.67284 203.728) (width 0.254) (layer F.Cu) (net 10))
 (segment (start 351.67284 203.728) (end 352.425 204.48016) (width 0.254) (layer F.Cu) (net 10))
 (segment (start 351.123 204.228) (end 352.17284 204.228) (width 0.254) (layer F.Cu) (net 10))
 (segment (start 352.17284 204.228) (end 352.425 204.48016) (width 0.254) (layer F.Cu) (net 10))
 (segment (start 351.123 205.228) (end 351.67716 205.228) (width 0.254) (layer F.Cu) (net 10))
 (segment (start 351.67716 205.228) (end 352.425 204.48016) (width 0.254) (layer F.Cu) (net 10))
 (segment (start 349.873 202.978) (end 349.873 201.69816) (width 0.254) (layer F.Cu) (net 11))
 (segment (start 349.873 201.69816) (end 349.89516 201.676) (width 0.254) (layer F.Cu) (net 11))
 (segment (start 349.373 206.978) (end 349.373 207.63084) (width 0.254) (layer F.Cu) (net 7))
 (segment (start 349.373 207.63084) (end 350.40316 208.661) (width 0.254) (layer F.Cu) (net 7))
 (segment (start 352.907598 208.153) (end 352.933 208.153) (width 0.254) (layer B.Cu) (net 2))
 (segment (start 345.952 204.728) (end 345.948 204.724) (width 0.254) (layer F.Cu) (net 2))
 (via (at 345.948 204.724) (size 0.889) (layers F.Cu B.Cu) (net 2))
 (segment (start 345.948 204.724) (end 345.948 207.772) (width 0.254) (layer B.Cu) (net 2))
 (segment (start 345.948 207.772) (end 346.329 208.153) (width 0.254) (layer B.Cu) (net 2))
 (segment (start 346.329 208.153) (end 352.907598 208.153) (width 0.254) (layer B.Cu) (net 2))
 (segment (start 347.123 204.728) (end 345.952 204.728) (width 0.254) (layer F.Cu) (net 2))
 (via (at 353.568 205.232) (size 0.889) (layers F.Cu B.Cu) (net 2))
 (segment (start 353.568 207.518) (end 353.568 205.232) (width 0.254) (layer B.Cu) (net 2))
 (segment (start 352.933 208.153) (end 353.568 207.518) (width 0.254) (layer B.Cu) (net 2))
 (segment (start 352.425 205.98384) (end 352.66884 205.98384) (width 0.254) (layer F.Cu) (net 2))
 (segment (start 352.425 205.98384) (end 352.81616 205.98384) (width 0.254) (layer F.Cu) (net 2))
 (segment (start 352.81616 205.98384) (end 353.568 205.232) (width 0.254) (layer F.Cu) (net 2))
 (segment (start 353.568 205.232) (end 355.6 203.2) (width 0.254) (layer F.Cu) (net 2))
 (segment (start 351.123 206.228) (end 352.18084 206.228) (width 0.254) (layer F.Cu) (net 2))
 (segment (start 352.18084 206.228) (end 352.425 205.98384) (width 0.254) (layer F.Cu) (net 2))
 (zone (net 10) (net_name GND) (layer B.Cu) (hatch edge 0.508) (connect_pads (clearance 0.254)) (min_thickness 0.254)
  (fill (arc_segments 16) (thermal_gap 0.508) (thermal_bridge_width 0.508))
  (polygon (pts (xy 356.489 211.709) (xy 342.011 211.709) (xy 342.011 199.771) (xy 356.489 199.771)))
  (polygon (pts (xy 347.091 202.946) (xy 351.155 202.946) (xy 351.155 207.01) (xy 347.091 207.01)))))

